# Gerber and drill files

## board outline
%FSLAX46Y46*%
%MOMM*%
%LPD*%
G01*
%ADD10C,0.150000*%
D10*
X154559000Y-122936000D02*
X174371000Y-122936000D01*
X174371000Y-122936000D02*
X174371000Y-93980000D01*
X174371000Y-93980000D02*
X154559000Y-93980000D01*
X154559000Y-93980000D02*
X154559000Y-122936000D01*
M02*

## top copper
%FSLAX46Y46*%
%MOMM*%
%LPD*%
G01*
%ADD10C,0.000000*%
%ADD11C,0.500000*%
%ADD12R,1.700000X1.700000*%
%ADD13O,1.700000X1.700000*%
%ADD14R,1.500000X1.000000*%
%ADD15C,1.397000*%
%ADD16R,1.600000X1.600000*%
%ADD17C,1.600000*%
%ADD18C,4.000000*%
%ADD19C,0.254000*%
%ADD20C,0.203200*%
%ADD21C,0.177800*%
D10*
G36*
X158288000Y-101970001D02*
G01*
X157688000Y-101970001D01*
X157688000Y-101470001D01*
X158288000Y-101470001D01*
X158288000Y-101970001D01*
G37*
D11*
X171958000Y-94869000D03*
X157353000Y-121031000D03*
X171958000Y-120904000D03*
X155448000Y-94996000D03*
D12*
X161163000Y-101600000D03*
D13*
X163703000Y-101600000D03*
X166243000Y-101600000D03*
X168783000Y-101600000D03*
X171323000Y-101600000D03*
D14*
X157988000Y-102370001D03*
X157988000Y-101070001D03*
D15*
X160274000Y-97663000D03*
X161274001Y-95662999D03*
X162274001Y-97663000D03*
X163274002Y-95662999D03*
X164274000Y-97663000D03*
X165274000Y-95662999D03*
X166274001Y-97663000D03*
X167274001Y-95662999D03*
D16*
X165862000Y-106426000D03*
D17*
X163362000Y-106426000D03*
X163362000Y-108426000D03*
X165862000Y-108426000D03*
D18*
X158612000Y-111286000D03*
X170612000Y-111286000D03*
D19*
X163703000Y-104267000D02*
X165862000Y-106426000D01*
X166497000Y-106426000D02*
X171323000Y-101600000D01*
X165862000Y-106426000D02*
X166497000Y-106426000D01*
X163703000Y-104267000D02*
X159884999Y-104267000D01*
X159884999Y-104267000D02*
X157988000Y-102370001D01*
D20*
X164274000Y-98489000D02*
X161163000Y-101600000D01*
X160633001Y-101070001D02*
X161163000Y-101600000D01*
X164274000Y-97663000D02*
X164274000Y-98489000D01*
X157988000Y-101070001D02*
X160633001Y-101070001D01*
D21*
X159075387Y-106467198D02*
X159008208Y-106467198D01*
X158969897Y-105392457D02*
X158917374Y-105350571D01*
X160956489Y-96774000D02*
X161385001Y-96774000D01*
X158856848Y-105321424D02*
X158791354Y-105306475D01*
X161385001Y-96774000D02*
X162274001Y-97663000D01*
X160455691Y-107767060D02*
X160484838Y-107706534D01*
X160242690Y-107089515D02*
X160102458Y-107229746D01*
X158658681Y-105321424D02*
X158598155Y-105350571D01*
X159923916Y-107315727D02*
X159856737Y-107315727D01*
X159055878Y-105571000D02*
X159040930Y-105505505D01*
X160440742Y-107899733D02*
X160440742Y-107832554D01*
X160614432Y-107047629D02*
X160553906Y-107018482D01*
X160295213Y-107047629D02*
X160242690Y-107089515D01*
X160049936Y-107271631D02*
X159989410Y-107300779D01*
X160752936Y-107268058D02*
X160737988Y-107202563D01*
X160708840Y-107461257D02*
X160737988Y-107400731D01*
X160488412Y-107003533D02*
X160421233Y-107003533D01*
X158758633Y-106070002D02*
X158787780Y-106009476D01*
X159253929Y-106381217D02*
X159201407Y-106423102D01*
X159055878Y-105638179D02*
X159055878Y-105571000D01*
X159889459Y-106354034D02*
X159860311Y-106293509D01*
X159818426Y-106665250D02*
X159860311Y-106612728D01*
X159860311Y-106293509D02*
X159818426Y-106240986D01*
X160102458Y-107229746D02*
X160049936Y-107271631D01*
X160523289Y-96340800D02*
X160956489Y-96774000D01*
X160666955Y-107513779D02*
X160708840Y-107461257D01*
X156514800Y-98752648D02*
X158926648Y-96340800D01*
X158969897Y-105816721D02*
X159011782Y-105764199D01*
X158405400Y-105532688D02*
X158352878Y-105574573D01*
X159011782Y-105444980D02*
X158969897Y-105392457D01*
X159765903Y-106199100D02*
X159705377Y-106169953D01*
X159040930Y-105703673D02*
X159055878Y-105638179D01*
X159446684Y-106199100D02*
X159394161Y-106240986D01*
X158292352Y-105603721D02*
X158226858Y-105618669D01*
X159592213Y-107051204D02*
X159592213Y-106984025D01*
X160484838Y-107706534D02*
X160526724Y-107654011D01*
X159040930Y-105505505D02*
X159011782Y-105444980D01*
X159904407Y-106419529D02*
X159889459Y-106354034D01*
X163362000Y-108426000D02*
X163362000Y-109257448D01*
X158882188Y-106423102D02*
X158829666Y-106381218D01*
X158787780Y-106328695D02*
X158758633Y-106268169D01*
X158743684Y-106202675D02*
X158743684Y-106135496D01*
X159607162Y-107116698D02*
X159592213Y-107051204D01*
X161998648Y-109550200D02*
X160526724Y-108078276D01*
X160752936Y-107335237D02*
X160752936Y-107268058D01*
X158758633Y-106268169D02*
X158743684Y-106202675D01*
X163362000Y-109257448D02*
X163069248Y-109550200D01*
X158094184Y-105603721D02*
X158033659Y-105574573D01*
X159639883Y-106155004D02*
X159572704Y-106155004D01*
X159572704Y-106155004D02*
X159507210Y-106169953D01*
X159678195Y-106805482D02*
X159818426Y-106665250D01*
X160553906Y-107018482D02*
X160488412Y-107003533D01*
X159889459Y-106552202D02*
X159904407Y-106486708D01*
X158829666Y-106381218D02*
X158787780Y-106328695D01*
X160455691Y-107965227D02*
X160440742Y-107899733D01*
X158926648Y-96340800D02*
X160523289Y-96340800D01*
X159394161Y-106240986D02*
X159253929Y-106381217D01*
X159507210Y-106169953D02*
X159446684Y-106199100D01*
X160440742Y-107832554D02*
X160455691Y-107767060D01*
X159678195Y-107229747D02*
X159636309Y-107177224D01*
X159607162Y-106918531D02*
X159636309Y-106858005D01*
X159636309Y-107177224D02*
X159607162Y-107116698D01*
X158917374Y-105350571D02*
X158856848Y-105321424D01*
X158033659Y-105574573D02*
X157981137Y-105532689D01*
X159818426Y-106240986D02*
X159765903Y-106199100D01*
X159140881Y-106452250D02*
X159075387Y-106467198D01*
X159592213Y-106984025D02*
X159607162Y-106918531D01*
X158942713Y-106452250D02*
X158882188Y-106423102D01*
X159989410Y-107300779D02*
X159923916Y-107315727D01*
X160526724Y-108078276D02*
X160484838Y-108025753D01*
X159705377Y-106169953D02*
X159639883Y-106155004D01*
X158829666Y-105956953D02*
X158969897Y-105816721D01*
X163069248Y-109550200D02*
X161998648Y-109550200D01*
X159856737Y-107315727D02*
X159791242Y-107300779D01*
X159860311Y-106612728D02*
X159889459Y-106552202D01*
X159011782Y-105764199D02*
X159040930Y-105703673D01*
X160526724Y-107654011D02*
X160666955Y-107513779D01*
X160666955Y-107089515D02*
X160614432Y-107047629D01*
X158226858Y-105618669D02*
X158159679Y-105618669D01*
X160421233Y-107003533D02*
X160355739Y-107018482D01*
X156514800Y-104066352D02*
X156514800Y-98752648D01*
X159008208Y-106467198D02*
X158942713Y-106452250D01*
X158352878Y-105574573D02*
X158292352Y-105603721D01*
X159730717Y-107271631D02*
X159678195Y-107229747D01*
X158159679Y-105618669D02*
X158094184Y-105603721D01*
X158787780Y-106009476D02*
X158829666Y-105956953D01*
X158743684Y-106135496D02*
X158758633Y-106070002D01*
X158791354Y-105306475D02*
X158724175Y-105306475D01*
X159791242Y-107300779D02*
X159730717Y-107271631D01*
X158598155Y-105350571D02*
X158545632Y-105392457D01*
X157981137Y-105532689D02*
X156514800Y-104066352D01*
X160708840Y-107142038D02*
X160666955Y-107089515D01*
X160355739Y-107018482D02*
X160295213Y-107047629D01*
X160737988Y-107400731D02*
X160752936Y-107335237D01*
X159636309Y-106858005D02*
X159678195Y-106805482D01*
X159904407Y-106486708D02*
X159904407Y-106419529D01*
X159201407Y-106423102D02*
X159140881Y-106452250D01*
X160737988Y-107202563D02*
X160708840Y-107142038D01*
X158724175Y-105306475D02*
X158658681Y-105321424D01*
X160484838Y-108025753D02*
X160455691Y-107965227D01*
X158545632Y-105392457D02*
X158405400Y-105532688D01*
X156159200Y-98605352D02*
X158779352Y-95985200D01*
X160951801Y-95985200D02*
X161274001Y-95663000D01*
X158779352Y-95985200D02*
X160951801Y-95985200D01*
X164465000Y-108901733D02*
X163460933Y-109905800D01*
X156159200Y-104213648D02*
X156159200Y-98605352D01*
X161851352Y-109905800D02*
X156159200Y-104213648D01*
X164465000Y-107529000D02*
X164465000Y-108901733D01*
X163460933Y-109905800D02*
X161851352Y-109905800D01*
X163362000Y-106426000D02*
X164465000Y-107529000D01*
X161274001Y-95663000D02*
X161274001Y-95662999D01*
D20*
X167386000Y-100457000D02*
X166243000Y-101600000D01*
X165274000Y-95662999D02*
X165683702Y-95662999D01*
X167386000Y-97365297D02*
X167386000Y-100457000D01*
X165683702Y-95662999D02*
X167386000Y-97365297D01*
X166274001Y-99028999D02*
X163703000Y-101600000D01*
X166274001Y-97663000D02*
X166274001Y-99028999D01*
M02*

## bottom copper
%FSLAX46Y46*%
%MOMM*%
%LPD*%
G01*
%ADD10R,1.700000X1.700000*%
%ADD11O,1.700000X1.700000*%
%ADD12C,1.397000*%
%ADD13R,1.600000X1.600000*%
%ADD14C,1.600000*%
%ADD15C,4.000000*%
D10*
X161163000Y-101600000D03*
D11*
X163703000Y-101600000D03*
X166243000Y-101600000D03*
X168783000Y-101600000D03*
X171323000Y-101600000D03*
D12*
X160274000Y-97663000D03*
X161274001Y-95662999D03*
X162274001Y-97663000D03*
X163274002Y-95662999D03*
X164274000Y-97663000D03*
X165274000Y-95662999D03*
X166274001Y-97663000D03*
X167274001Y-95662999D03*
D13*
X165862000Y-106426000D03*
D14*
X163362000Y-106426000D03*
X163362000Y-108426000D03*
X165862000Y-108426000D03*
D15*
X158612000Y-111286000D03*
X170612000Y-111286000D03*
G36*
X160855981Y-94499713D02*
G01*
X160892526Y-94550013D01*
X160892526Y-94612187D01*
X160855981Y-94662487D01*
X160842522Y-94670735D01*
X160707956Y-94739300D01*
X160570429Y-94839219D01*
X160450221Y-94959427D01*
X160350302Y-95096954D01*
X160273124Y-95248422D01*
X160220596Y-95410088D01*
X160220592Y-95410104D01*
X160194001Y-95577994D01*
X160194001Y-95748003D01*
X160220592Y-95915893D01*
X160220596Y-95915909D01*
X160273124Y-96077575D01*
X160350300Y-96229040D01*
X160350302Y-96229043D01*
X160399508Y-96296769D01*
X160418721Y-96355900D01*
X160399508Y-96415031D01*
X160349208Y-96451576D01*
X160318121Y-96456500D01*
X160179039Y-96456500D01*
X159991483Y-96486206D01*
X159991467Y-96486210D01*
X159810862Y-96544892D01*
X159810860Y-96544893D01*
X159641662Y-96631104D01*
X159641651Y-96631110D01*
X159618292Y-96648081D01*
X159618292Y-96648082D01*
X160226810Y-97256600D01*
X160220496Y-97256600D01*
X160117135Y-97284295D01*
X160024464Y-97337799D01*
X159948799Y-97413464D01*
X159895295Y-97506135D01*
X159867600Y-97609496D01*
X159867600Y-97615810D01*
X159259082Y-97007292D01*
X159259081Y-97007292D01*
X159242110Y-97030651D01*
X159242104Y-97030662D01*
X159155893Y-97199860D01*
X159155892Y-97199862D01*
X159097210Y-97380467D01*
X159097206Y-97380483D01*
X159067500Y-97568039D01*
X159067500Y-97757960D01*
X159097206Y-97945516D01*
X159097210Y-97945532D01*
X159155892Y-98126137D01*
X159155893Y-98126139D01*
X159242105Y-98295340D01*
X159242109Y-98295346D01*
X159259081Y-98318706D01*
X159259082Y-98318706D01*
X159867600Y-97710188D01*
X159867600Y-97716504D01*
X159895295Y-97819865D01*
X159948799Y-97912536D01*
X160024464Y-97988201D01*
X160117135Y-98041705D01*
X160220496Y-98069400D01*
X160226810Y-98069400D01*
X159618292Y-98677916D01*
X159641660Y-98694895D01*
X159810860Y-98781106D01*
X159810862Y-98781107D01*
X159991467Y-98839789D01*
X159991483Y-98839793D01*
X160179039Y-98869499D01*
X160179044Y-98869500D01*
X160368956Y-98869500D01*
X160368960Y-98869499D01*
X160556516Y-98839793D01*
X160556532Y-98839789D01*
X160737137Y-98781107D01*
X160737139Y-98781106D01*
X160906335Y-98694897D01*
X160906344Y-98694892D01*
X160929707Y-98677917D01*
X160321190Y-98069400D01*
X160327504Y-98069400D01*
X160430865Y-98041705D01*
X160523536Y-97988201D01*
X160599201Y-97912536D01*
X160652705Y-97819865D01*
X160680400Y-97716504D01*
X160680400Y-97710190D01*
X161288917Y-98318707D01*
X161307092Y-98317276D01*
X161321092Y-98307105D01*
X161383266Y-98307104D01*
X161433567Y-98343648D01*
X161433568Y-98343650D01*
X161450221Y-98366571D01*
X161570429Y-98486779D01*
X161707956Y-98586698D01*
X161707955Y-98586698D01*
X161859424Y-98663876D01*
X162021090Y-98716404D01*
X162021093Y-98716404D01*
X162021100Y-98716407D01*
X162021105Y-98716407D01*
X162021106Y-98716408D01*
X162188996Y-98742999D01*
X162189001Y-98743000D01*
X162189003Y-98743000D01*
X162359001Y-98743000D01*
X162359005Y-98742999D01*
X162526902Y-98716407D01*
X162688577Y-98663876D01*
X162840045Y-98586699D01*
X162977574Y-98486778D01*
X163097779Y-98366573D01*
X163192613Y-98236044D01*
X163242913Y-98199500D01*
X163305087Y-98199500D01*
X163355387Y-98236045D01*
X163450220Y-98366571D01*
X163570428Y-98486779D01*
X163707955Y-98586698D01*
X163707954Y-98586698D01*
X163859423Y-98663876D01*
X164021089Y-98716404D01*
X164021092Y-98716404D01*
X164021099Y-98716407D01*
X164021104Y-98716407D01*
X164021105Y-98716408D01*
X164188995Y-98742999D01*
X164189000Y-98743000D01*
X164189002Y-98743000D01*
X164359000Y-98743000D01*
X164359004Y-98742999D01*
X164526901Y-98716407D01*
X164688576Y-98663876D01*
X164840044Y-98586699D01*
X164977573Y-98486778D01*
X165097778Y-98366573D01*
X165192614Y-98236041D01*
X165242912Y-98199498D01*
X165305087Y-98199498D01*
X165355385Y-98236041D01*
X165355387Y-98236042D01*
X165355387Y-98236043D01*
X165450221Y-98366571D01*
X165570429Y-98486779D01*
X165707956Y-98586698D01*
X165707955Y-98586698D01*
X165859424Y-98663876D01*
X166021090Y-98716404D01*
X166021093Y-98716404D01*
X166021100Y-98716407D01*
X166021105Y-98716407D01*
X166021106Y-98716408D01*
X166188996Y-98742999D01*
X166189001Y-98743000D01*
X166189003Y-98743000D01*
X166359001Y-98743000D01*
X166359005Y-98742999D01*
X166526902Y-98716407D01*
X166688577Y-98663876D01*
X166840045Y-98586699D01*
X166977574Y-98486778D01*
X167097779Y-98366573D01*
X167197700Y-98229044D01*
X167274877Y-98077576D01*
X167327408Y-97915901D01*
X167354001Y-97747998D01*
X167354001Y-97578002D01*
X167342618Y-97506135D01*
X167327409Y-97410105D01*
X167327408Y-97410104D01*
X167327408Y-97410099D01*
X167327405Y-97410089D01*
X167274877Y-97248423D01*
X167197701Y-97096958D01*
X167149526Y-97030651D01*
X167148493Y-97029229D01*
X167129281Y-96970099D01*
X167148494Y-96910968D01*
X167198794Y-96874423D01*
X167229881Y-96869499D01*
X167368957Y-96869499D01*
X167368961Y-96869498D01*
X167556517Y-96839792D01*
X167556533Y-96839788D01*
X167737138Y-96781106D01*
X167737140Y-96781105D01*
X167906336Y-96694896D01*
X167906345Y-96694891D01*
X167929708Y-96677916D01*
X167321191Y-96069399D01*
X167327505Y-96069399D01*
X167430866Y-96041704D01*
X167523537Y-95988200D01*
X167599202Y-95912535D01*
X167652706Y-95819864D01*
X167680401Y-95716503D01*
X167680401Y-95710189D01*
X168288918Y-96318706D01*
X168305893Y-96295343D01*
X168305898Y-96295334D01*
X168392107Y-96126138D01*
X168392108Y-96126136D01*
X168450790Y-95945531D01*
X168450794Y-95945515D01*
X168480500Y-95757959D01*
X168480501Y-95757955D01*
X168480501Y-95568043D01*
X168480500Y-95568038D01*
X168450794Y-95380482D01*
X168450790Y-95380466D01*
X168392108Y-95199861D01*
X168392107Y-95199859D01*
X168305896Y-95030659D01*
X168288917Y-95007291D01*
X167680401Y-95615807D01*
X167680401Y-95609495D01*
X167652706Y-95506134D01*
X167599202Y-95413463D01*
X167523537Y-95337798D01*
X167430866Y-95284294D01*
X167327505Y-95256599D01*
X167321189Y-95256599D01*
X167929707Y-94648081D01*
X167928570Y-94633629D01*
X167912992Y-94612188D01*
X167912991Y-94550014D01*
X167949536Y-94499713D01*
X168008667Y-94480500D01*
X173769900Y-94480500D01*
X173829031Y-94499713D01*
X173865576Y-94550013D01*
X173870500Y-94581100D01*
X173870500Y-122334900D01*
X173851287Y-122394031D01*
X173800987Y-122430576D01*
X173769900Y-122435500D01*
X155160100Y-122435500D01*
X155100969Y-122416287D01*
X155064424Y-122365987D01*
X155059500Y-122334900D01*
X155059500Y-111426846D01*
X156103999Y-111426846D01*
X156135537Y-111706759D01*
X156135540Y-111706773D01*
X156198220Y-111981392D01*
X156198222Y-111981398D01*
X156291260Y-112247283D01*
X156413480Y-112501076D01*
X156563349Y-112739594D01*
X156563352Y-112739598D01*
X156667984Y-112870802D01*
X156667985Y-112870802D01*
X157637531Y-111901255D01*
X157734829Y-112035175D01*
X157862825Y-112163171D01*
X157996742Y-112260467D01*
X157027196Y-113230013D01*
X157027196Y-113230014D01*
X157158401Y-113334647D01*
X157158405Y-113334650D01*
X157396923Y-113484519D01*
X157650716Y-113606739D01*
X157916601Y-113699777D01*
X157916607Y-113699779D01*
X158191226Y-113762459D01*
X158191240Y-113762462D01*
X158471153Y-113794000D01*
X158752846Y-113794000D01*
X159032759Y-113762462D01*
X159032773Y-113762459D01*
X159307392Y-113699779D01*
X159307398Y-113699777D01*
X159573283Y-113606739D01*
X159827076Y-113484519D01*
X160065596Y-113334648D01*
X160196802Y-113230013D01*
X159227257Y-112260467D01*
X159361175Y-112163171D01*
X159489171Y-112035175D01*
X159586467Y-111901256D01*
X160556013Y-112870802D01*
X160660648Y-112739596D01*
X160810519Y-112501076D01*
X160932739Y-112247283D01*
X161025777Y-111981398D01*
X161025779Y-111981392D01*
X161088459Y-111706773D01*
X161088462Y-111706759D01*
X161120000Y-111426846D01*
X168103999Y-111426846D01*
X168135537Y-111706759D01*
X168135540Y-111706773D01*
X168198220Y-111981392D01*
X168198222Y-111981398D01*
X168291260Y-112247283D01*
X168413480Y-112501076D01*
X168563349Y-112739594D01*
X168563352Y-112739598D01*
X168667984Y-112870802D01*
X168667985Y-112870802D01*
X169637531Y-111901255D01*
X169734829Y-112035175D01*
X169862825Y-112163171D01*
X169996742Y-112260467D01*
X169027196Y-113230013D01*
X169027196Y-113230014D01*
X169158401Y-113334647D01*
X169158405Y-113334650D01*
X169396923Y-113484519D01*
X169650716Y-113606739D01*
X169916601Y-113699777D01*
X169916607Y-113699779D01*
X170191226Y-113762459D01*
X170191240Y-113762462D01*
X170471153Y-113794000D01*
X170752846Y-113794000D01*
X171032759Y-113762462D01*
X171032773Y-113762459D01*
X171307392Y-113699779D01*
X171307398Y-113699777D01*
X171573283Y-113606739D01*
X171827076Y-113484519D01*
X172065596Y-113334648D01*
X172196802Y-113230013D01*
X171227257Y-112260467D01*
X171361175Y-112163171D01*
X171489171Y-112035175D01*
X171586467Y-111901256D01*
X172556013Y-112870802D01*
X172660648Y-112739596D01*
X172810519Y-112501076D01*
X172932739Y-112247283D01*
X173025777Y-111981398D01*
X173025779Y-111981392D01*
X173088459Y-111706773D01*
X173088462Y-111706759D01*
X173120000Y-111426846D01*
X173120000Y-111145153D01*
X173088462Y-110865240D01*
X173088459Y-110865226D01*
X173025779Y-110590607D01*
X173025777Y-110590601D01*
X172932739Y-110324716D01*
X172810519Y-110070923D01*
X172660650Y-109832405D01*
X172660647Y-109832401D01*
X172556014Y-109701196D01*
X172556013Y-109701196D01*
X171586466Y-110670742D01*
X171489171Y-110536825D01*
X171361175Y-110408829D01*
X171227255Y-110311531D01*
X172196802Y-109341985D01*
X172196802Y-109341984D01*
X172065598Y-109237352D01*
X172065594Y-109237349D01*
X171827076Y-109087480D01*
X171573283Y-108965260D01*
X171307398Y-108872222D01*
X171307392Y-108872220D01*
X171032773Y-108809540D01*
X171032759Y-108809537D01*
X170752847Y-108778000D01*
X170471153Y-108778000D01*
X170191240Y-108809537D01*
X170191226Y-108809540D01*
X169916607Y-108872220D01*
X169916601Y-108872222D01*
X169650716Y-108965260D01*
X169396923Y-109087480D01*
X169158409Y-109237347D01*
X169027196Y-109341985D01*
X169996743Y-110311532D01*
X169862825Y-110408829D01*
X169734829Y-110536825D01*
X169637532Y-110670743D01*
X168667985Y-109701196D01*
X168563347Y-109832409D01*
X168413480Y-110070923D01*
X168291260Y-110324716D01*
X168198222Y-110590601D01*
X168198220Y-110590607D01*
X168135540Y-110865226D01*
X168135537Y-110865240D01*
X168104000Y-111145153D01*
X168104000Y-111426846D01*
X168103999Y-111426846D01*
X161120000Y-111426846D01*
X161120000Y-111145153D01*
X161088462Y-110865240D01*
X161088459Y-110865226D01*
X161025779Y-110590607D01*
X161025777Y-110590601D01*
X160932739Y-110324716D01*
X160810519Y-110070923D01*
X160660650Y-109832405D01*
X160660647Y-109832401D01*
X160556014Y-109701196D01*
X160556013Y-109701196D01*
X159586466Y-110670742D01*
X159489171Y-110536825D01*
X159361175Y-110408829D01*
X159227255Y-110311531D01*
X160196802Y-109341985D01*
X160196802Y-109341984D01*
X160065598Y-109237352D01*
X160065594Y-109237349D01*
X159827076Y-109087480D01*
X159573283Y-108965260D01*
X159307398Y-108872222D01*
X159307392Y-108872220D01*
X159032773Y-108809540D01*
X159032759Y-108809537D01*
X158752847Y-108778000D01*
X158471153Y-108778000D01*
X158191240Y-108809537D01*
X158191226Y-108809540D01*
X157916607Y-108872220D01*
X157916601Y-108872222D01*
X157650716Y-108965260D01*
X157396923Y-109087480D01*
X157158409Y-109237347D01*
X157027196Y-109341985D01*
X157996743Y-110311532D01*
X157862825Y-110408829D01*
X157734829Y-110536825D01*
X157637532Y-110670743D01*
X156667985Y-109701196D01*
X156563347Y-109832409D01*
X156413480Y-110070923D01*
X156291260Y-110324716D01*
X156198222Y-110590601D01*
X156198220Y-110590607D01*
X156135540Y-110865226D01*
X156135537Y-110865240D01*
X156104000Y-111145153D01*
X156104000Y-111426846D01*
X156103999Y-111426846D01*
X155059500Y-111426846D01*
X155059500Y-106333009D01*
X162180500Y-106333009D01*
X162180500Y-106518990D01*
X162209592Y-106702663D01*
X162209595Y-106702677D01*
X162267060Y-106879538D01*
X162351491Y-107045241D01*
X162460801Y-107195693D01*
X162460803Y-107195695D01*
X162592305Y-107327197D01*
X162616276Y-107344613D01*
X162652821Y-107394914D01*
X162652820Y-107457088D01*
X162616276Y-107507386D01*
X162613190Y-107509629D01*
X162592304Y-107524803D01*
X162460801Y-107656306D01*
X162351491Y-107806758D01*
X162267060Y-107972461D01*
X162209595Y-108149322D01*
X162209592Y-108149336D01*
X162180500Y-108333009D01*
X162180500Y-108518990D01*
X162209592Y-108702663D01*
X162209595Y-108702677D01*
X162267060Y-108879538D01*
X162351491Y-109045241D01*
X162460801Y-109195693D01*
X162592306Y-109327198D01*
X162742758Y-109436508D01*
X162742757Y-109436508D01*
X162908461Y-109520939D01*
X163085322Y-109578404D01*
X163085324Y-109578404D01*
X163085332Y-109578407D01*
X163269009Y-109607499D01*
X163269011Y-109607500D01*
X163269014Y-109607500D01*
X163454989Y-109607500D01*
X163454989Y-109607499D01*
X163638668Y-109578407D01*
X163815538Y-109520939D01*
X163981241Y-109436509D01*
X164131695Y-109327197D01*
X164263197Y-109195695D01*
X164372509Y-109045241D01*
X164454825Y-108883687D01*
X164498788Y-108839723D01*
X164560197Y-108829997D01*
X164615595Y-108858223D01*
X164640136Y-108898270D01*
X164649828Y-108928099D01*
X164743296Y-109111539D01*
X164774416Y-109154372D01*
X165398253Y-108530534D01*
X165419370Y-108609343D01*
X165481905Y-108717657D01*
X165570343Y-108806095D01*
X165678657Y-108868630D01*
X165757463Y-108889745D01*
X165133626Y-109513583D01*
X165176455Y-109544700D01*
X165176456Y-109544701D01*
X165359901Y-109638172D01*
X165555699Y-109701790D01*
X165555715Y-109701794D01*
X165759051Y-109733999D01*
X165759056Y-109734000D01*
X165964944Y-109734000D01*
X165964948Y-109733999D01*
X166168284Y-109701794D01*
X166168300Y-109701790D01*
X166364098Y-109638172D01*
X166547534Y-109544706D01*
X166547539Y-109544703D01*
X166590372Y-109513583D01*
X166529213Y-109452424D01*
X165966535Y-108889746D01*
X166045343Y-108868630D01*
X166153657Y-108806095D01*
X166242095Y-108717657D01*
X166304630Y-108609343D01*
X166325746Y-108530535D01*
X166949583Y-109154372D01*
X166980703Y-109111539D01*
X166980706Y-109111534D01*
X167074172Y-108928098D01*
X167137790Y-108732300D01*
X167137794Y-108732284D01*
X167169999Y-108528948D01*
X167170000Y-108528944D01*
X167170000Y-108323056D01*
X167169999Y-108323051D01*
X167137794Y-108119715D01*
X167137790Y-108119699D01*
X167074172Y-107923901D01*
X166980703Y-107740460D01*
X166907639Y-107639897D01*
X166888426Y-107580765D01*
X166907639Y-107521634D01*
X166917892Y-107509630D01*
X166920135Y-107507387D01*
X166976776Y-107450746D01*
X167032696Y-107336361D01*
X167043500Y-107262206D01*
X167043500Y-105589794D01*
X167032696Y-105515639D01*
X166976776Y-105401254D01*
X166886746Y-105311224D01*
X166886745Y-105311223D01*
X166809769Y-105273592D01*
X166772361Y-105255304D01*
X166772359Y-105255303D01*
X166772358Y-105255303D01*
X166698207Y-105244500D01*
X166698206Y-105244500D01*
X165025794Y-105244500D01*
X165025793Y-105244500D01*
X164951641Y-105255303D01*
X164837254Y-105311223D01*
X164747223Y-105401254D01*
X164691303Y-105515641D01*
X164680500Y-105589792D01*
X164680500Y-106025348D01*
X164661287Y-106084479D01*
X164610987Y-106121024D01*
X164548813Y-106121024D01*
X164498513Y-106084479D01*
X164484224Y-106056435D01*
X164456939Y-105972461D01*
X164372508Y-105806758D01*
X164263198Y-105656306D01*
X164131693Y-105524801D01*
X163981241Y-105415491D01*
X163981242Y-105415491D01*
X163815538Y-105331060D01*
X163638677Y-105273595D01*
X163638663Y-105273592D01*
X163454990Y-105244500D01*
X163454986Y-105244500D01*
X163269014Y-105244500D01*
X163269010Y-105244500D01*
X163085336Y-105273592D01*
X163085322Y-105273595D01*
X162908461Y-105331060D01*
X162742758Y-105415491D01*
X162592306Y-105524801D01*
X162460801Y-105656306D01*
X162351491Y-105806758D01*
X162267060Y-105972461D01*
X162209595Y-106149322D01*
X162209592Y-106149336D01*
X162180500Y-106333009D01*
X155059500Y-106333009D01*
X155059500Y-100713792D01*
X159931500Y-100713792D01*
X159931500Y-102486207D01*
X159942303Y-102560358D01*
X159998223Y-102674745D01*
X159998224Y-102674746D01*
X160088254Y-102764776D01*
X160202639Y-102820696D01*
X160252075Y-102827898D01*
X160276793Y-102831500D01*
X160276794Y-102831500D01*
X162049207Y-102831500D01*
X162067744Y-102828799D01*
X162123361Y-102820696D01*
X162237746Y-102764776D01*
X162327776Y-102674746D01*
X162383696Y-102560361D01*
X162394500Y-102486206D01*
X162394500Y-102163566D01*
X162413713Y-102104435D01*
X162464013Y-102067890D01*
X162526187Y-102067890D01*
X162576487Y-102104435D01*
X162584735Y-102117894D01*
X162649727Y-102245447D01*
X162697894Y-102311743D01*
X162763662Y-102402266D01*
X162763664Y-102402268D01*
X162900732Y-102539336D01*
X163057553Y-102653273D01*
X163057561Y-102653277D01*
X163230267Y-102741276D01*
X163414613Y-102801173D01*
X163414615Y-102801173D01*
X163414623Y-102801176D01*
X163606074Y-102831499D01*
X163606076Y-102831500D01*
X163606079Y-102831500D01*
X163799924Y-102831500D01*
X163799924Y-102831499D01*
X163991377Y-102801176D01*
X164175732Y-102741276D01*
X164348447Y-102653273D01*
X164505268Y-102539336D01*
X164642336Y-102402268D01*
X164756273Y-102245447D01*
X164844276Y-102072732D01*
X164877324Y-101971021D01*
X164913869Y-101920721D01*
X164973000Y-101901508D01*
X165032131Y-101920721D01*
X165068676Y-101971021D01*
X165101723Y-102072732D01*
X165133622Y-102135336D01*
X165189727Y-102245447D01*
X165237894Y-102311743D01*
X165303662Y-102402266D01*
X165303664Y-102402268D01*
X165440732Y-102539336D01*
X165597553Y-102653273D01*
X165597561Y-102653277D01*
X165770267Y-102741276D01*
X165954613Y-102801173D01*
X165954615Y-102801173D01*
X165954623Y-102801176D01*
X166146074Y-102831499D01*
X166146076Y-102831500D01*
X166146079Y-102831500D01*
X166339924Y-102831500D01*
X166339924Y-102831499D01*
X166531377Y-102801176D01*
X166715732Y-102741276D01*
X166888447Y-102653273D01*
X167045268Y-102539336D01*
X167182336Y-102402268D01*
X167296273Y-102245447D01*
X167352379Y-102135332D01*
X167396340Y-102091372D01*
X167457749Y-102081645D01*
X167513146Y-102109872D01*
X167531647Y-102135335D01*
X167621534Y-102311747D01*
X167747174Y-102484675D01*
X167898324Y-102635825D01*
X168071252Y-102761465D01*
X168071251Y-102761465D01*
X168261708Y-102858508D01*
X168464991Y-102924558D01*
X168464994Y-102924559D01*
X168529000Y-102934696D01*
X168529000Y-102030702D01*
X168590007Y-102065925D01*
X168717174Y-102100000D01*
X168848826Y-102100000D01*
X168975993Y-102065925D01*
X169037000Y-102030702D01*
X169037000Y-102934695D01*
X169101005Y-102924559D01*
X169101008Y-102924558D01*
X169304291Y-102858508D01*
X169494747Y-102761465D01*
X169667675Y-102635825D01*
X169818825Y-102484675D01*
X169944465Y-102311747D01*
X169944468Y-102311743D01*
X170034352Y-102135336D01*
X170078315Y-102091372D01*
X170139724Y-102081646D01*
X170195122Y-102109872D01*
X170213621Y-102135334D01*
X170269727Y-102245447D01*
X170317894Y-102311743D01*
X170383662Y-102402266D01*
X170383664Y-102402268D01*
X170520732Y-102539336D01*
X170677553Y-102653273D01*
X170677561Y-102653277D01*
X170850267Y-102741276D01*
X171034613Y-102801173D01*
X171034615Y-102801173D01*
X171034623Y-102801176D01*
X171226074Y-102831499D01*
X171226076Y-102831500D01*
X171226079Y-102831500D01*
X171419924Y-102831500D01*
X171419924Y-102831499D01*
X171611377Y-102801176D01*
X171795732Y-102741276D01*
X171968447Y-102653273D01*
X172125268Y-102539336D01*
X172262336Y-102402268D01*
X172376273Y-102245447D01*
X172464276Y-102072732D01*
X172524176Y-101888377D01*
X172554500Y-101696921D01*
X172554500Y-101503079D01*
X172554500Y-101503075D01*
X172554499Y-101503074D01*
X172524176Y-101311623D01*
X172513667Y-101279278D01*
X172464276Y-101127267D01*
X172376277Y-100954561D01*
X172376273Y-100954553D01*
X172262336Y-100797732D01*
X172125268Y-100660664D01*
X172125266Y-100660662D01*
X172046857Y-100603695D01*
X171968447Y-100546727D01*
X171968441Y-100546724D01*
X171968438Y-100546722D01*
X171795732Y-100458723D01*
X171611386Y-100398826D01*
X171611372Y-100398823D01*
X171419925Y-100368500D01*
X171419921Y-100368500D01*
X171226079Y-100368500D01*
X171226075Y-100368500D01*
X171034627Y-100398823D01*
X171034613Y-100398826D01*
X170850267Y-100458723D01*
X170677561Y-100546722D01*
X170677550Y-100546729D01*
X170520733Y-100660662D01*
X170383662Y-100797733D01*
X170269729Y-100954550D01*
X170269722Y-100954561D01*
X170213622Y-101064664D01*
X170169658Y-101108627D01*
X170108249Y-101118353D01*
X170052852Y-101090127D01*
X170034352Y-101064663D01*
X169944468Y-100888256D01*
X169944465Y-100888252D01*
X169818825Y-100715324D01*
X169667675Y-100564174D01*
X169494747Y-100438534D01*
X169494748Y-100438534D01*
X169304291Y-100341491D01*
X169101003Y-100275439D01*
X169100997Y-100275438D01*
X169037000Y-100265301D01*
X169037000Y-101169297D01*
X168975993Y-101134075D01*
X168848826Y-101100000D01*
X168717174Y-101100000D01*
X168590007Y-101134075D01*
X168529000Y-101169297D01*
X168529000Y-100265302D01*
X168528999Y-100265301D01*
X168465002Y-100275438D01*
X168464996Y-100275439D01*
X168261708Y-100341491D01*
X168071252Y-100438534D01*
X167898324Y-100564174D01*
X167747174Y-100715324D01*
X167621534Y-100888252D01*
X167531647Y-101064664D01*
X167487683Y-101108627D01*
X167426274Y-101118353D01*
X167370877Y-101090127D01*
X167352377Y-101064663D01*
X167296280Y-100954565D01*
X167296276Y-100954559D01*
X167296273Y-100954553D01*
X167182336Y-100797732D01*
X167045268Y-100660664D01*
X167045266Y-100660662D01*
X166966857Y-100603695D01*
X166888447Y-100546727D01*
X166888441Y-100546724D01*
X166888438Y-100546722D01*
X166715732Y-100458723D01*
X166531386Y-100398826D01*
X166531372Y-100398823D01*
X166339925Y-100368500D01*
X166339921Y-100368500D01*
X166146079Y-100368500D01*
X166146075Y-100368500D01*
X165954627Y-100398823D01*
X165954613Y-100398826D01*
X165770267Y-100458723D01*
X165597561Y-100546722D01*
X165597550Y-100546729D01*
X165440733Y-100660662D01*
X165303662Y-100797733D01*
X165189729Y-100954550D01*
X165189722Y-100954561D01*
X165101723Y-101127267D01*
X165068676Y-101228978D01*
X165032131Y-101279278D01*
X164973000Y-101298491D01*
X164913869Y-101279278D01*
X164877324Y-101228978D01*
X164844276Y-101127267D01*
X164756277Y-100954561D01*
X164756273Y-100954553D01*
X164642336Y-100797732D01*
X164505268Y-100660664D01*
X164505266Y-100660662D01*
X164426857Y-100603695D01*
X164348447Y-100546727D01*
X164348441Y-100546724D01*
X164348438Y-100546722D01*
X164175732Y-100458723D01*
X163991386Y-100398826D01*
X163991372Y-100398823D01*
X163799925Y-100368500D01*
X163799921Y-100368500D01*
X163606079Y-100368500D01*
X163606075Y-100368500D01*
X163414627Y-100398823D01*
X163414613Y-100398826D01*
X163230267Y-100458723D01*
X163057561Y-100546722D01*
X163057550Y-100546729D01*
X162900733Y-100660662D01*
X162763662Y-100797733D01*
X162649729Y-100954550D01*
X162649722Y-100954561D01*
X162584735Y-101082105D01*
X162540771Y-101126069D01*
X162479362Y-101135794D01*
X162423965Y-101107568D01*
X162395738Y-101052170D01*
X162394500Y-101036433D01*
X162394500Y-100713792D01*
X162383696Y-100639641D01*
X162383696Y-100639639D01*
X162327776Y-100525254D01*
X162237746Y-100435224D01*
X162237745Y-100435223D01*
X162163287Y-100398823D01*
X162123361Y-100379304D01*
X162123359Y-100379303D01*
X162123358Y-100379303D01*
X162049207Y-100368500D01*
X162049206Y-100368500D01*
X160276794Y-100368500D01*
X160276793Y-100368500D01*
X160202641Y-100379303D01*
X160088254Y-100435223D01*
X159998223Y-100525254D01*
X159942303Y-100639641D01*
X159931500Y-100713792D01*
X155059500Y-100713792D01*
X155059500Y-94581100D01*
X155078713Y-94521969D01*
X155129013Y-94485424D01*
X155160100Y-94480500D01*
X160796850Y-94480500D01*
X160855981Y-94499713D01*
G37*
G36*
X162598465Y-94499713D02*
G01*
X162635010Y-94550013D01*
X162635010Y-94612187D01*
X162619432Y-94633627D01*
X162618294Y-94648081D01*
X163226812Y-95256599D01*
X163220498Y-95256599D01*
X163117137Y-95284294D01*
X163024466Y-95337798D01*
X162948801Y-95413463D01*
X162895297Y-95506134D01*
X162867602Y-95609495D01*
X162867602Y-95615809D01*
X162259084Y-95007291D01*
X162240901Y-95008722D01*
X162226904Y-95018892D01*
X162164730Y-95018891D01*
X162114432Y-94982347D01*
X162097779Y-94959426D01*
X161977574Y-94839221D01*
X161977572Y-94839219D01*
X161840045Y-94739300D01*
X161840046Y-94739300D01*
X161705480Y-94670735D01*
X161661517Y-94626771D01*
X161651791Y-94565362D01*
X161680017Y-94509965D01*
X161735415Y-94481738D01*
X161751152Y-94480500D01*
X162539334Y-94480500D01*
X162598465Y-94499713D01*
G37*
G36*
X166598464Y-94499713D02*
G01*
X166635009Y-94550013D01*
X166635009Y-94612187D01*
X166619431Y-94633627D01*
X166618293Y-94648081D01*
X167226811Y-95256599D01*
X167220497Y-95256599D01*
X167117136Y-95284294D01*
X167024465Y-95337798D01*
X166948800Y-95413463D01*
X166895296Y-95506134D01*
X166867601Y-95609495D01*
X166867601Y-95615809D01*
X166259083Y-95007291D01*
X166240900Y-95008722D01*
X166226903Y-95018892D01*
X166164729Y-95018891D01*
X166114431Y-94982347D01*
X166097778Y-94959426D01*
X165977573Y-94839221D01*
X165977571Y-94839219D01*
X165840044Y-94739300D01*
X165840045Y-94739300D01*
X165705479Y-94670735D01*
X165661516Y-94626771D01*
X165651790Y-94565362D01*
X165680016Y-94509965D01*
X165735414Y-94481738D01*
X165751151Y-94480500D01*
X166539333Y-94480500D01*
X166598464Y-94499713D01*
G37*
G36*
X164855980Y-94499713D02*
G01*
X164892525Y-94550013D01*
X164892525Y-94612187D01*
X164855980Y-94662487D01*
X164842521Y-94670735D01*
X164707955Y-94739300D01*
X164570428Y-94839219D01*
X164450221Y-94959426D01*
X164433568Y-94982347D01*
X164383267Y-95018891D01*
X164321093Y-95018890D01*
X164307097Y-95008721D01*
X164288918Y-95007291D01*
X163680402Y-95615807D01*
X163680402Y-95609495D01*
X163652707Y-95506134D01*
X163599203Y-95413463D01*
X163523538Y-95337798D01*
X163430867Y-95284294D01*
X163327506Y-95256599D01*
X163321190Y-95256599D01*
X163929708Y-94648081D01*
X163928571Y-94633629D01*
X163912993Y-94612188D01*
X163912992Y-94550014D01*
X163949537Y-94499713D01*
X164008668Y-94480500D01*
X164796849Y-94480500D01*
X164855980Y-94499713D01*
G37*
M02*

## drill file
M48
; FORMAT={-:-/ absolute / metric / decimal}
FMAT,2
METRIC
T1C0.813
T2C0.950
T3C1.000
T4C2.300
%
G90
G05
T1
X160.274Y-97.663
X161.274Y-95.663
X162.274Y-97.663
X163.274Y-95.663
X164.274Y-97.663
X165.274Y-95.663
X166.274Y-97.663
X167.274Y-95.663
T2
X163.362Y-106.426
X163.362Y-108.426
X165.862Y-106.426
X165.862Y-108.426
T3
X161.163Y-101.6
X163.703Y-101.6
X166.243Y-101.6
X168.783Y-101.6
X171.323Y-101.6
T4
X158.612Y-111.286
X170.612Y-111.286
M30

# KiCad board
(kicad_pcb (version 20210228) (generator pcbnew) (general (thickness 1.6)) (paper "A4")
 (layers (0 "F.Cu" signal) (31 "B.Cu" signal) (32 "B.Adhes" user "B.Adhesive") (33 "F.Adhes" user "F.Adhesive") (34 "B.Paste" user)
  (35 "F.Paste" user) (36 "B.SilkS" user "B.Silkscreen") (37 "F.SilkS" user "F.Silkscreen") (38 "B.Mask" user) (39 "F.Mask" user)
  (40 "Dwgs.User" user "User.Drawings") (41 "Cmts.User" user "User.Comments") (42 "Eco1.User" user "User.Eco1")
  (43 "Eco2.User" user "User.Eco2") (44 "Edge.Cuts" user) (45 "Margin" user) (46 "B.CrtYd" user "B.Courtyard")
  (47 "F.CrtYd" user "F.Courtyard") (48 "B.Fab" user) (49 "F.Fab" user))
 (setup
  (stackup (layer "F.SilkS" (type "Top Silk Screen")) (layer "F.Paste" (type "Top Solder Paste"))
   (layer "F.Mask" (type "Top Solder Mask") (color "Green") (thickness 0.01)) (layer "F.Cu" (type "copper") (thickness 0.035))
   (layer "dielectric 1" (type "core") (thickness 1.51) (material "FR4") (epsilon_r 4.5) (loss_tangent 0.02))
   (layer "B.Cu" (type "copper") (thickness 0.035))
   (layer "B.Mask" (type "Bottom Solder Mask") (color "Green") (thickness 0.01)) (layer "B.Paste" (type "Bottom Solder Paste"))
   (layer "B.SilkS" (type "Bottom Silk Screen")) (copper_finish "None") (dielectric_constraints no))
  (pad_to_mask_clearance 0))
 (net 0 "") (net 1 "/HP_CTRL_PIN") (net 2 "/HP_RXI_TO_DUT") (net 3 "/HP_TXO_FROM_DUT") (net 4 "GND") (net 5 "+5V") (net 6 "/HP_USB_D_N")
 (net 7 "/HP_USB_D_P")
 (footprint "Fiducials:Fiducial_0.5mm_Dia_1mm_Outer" (layer "F.Cu") (at 171.958 94.869)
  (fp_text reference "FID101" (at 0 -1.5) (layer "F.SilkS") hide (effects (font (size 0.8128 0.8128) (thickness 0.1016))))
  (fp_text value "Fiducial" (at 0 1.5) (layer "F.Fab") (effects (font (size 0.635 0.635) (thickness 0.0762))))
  (pad "~" smd circle (at 0 0) (locked) (size 0.5 0.5) (layers "F.Cu" "F.Mask") (solder_mask_margin 0.25) (clearance 0.25)))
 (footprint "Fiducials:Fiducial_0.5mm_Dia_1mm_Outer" (layer "F.Cu") (at 157.353 121.031)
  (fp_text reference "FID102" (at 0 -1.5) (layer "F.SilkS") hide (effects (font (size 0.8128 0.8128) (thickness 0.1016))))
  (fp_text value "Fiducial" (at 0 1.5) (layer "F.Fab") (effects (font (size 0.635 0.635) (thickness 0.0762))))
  (pad "~" smd circle (at 0 0) (locked) (size 0.5 0.5) (layers "F.Cu" "F.Mask") (solder_mask_margin 0.25) (clearance 0.25)))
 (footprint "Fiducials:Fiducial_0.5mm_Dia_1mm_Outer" (layer "F.Cu") (at 171.958 120.904)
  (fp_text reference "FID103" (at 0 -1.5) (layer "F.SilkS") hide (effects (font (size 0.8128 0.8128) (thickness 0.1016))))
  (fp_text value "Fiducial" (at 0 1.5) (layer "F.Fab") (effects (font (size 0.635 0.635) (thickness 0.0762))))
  (pad "~" smd circle (at 0 0) (locked) (size 0.5 0.5) (layers "F.Cu" "F.Mask") (solder_mask_margin 0.25) (clearance 0.25)))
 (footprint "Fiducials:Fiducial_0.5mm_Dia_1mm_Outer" (layer "F.Cu") (at 155.448 94.996)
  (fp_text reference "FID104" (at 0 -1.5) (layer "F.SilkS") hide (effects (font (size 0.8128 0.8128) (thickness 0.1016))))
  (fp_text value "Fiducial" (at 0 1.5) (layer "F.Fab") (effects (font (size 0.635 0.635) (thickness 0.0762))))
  (pad "~" smd circle (at 0 0) (locked) (size 0.5 0.5) (layers "F.Cu" "F.Mask") (solder_mask_margin 0.25) (clearance 0.25)))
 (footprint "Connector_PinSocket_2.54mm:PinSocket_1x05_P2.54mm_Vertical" (layer "F.Cu") (at 161.163 101.6 90)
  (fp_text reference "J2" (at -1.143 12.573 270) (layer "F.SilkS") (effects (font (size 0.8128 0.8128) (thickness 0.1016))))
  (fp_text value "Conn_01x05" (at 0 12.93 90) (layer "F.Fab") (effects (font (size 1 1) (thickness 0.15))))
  (pad "1" thru_hole rect (at 0 0 90) (locked) (size 1.7 1.7) (drill 1) (layers *.Cu *.Mask) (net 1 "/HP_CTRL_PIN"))
  (pad "2" thru_hole oval (at 0 2.54 90) (locked) (size 1.7 1.7) (drill 1) (layers *.Cu *.Mask) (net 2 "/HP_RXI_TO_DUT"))
  (pad "3" thru_hole oval (at 0 5.08 90) (locked) (size 1.7 1.7) (drill 1) (layers *.Cu *.Mask) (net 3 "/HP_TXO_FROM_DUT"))
  (pad "4" thru_hole oval (at 0 7.62 90) (locked) (size 1.7 1.7) (drill 1) (layers *.Cu *.Mask) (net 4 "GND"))
  (pad "5" thru_hole oval (at 0 10.16 90) (locked) (size 1.7 1.7) (drill 1) (layers *.Cu *.Mask) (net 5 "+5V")))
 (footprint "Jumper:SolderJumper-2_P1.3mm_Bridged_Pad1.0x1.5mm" (layer "F.Cu") (at 157.988 101.720001 90)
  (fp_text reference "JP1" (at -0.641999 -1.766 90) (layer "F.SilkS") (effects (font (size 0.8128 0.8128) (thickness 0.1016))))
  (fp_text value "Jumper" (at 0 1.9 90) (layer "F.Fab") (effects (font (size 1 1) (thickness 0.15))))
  (fp_poly (pts (xy -0.25 -0.3) (xy 0.25 -0.3) (xy 0.25 0.3) (xy -0.25 0.3)) (layer "F.Cu") (width 0) (fill solid))
  (pad "1" smd rect (at -0.65 0 90) (locked) (size 1 1.5) (layers "F.Cu" "F.Mask") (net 5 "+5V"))
  (pad "2" smd rect (at 0.65 0 90) (locked) (size 1 1.5) (layers "F.Cu" "F.Mask") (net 1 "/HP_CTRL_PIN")))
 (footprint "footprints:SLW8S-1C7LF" (layer "F.Cu") (at 160.274 97.663)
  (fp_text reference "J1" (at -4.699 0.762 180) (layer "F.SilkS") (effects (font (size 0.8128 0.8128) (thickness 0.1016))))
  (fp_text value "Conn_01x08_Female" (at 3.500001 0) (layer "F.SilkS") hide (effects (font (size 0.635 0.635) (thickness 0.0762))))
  (pad "1" thru_hole circle (at 0 0) (locked) (size 1.397 1.397) (drill 0.8128) (layers *.Cu *.Mask) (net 4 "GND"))
  (pad "2" thru_hole circle (at 1.000001 -2.000001) (locked) (size 1.397 1.397) (drill 0.8128) (layers *.Cu *.Mask) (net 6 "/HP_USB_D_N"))
  (pad "3" thru_hole circle (at 2.000001 0) (locked) (size 1.397 1.397) (drill 0.8128) (layers *.Cu *.Mask) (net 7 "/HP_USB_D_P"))
  (pad "4" thru_hole circle (at 3.000002 -2.000001) (locked) (size 1.397 1.397) (drill 0.8128) (layers *.Cu *.Mask) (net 4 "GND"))
  (pad "5" thru_hole circle (at 4 0) (locked) (size 1.397 1.397) (drill 0.8128) (layers *.Cu *.Mask) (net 1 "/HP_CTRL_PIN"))
  (pad "6" thru_hole circle (at 5 -2.000001) (locked) (size 1.397 1.397) (drill 0.8128) (layers *.Cu *.Mask) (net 3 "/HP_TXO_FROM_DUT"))
  (pad "7" thru_hole circle (at 6.000001 0) (locked) (size 1.397 1.397) (drill 0.8128) (layers *.Cu *.Mask) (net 2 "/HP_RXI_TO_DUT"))
  (pad "8" thru_hole circle (at 7.000001 -2.000001) (locked) (size 1.397 1.397) (drill 0.8128) (layers *.Cu *.Mask) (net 4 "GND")))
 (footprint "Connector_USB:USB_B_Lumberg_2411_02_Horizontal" (layer "F.Cu") (at 165.862 106.426 -90)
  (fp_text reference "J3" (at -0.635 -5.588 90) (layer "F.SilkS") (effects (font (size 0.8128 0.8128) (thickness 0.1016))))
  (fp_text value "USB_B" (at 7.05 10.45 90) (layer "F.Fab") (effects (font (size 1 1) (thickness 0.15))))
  (pad "1" thru_hole rect (at 0 0) (locked) (size 1.6 1.6) (drill 0.95) (layers *.Cu *.Mask) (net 5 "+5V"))
  (pad "2" thru_hole circle (at 0 2.5) (locked) (size 1.6 1.6) (drill 0.95) (layers *.Cu *.Mask) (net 6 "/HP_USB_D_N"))
  (pad "3" thru_hole circle (at 2 2.5) (locked) (size 1.6 1.6) (drill 0.95) (layers *.Cu *.Mask) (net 7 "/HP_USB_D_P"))
  (pad "4" thru_hole circle (at 2 0) (locked) (size 1.6 1.6) (drill 0.95) (layers *.Cu *.Mask) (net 4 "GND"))
  (pad "5" thru_hole circle (at 4.86 7.25) (locked) (size 4 4) (drill 2.3) (layers *.Cu *.Mask) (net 4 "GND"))
  (pad "5" thru_hole circle (at 4.86 -4.75) (locked) (size 4 4) (drill 2.3) (layers *.Cu *.Mask) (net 4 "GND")))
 (gr_line (start 154.559 122.936) (end 174.371 122.936) (layer "Edge.Cuts") (width 0.15))
 (gr_line (start 174.371 122.936) (end 174.371 93.98) (layer "Edge.Cuts") (width 0.15))
 (gr_line (start 174.371 93.98) (end 154.559 93.98) (layer "Edge.Cuts") (width 0.15))
 (gr_line (start 154.559 93.98) (end 154.559 122.936) (layer "Edge.Cuts") (width 0.15))
 (segment (start 163.703 104.267) (end 165.862 106.426) (width 0.254) (layer "F.Cu") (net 5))
 (segment (start 166.497 106.426) (end 171.323 101.6) (width 0.254) (layer "F.Cu") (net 5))
 (segment (start 165.862 106.426) (end 166.497 106.426) (width 0.254) (layer "F.Cu") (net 5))
 (segment (start 163.703 104.267) (end 159.884999 104.267) (width 0.254) (layer "F.Cu") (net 5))
 (segment (start 159.884999 104.267) (end 157.988 102.370001) (width 0.254) (layer "F.Cu") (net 5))
 (segment (start 164.274 98.489) (end 161.163 101.6) (width 0.2032) (layer "F.Cu") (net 1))
 (segment (start 160.633001 101.070001) (end 161.163 101.6) (width 0.2032) (layer "F.Cu") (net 1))
 (segment (start 164.274 97.663) (end 164.274 98.489) (width 0.2032) (layer "F.Cu") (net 1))
 (segment (start 157.988 101.070001) (end 160.633001 101.070001) (width 0.2032) (layer "F.Cu") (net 1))
 (segment (start 159.075387 106.467198) (end 159.008208 106.467198) (width 0.1778) (layer "F.Cu") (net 7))
 (segment (start 158.969897 105.392457) (end 158.917374 105.350571) (width 0.1778) (layer "F.Cu") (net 7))
 (segment (start 160.956489 96.774) (end 161.385001 96.774) (width 0.1778) (layer "F.Cu") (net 7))
 (segment (start 158.856848 105.321424) (end 158.791354 105.306475) (width 0.1778) (layer "F.Cu") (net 7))
 (segment (start 161.385001 96.774) (end 162.274001 97.663) (width 0.1778) (layer "F.Cu") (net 7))
 (segment (start 160.455691 107.76706) (end 160.484838 107.706534) (width 0.1778) (layer "F.Cu") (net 7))
 (segment (start 160.24269 107.089515) (end 160.102458 107.229746) (width 0.1778) (layer "F.Cu") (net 7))
 (segment (start 158.658681 105.321424) (end 158.598155 105.350571) (width 0.1778) (layer "F.Cu") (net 7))
 (segment (start 159.923916 107.315727) (end 159.856737 107.315727) (width 0.1778) (layer "F.Cu") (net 7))
 (segment (start 159.055878 105.571) (end 159.04093 105.505505) (width 0.1778) (layer "F.Cu") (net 7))
 (segment (start 160.440742 107.899733) (end 160.440742 107.832554) (width 0.1778) (layer "F.Cu") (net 7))
 (segment (start 160.614432 107.047629) (end 160.553906 107.018482) (width 0.1778) (layer "F.Cu") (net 7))
 (segment (start 160.295213 107.047629) (end 160.24269 107.089515) (width 0.1778) (layer "F.Cu") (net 7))
 (segment (start 160.049936 107.271631) (end 159.98941 107.300779) (width 0.1778) (layer "F.Cu") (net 7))
 (segment (start 160.752936 107.268058) (end 160.737988 107.202563) (width 0.1778) (layer "F.Cu") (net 7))
 (segment (start 160.70884 107.461257) (end 160.737988 107.400731) (width 0.1778) (layer "F.Cu") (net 7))
 (segment (start 160.488412 107.003533) (end 160.421233 107.003533) (width 0.1778) (layer "F.Cu") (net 7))
 (segment (start 158.758633 106.070002) (end 158.78778 106.009476) (width 0.1778) (layer "F.Cu") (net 7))
 (segment (start 159.253929 106.381217) (end 159.201407 106.423102) (width 0.1778) (layer "F.Cu") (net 7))
 (segment (start 159.055878 105.638179) (end 159.055878 105.571) (width 0.1778) (layer "F.Cu") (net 7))
 (segment (start 159.889459 106.354034) (end 159.860311 106.293509) (width 0.1778) (layer "F.Cu") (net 7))
 (segment (start 159.818426 106.66525) (end 159.860311 106.612728) (width 0.1778) (layer "F.Cu") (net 7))
 (segment (start 159.860311 106.293509) (end 159.818426 106.240986) (width 0.1778) (layer "F.Cu") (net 7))
 (segment (start 160.102458 107.229746) (end 160.049936 107.271631) (width 0.1778) (layer "F.Cu") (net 7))
 (segment (start 160.523289 96.3408) (end 160.956489 96.774) (width 0.1778) (layer "F.Cu") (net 7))
 (segment (start 160.666955 107.513779) (end 160.70884 107.461257) (width 0.1778) (layer "F.Cu") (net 7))
 (segment (start 156.5148 98.752648) (end 158.926648 96.3408) (width 0.1778) (layer "F.Cu") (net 7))
 (segment (start 158.969897 105.816721) (end 159.011782 105.764199) (width 0.1778) (layer "F.Cu") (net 7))
 (segment (start 158.4054 105.532688) (end 158.352878 105.574573) (width 0.1778) (layer "F.Cu") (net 7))
 (segment (start 159.011782 105.44498) (end 158.969897 105.392457) (width 0.1778) (layer "F.Cu") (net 7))
 (segment (start 159.765903 106.1991) (end 159.705377 106.169953) (width 0.1778) (layer "F.Cu") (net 7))
 (segment (start 159.04093 105.703673) (end 159.055878 105.638179) (width 0.1778) (layer "F.Cu") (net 7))
 (segment (start 159.446684 106.1991) (end 159.394161 106.240986) (width 0.1778) (layer "F.Cu") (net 7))
 (segment (start 158.292352 105.603721) (end 158.226858 105.618669) (width 0.1778) (layer "F.Cu") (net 7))
 (segment (start 159.592213 107.051204) (end 159.592213 106.984025) (width 0.1778) (layer "F.Cu") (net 7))
 (segment (start 160.484838 107.706534) (end 160.526724 107.654011) (width 0.1778) (layer "F.Cu") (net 7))
 (segment (start 159.04093 105.505505) (end 159.011782 105.44498) (width 0.1778) (layer "F.Cu") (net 7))
 (segment (start 159.904407 106.419529) (end 159.889459 106.354034) (width 0.1778) (layer "F.Cu") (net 7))
 (segment (start 163.362 108.426) (end 163.362 109.257448) (width 0.1778) (layer "F.Cu") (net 7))
 (segment (start 158.882188 106.423102) (end 158.829666 106.381218) (width 0.1778) (layer "F.Cu") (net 7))
 (segment (start 158.78778 106.328695) (end 158.758633 106.268169) (width 0.1778) (layer "F.Cu") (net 7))
 (segment (start 158.743684 106.202675) (end 158.743684 106.135496) (width 0.1778) (layer "F.Cu") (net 7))
 (segment (start 159.607162 107.116698) (end 159.592213 107.051204) (width 0.1778) (layer "F.Cu") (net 7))
 (segment (start 161.998648 109.5502) (end 160.526724 108.078276) (width 0.1778) (layer "F.Cu") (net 7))
 (segment (start 160.752936 107.335237) (end 160.752936 107.268058) (width 0.1778) (layer "F.Cu") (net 7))
 (segment (start 158.758633 106.268169) (end 158.743684 106.202675) (width 0.1778) (layer "F.Cu") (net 7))
 (segment (start 163.362 109.257448) (end 163.069248 109.5502) (width 0.1778) (layer "F.Cu") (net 7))
 (segment (start 158.094184 105.603721) (end 158.033659 105.574573) (width 0.1778) (layer "F.Cu") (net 7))
 (segment (start 159.639883 106.155004) (end 159.572704 106.155004) (width 0.1778) (layer "F.Cu") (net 7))
 (segment (start 159.572704 106.155004) (end 159.50721 106.169953) (width 0.1778) (layer "F.Cu") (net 7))
 (segment (start 159.678195 106.805482) (end 159.818426 106.66525) (width 0.1778) (layer "F.Cu") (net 7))
 (segment (start 160.553906 107.018482) (end 160.488412 107.003533) (width 0.1778) (layer "F.Cu") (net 7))
 (segment (start 159.889459 106.552202) (end 159.904407 106.486708) (width 0.1778) (layer "F.Cu") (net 7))
 (segment (start 158.829666 106.381218) (end 158.78778 106.328695) (width 0.1778) (layer "F.Cu") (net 7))
 (segment (start 160.455691 107.965227) (end 160.440742 107.899733) (width 0.1778) (layer "F.Cu") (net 7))
 (segment (start 158.926648 96.3408) (end 160.523289 96.3408) (width 0.1778) (layer "F.Cu") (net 7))
 (segment (start 159.394161 106.240986) (end 159.253929 106.381217) (width 0.1778) (layer "F.Cu") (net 7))
 (segment (start 159.50721 106.169953) (end 159.446684 106.1991) (width 0.1778) (layer "F.Cu") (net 7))
 (segment (start 160.440742 107.832554) (end 160.455691 107.76706) (width 0.1778) (layer "F.Cu") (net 7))
 (segment (start 159.678195 107.229747) (end 159.636309 107.177224) (width 0.1778) (layer "F.Cu") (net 7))
 (segment (start 159.607162 106.918531) (end 159.636309 106.858005) (width 0.1778) (layer "F.Cu") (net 7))
 (segment (start 159.636309 107.177224) (end 159.607162 107.116698) (width 0.1778) (layer "F.Cu") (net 7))
 (segment (start 158.917374 105.350571) (end 158.856848 105.321424) (width 0.1778) (layer "F.Cu") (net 7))
 (segment (start 158.033659 105.574573) (end 157.981137 105.532689) (width 0.1778) (layer "F.Cu") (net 7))
 (segment (start 159.818426 106.240986) (end 159.765903 106.1991) (width 0.1778) (layer "F.Cu") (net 7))
 (segment (start 159.140881 106.45225) (end 159.075387 106.467198) (width 0.1778) (layer "F.Cu") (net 7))
 (segment (start 159.592213 106.984025) (end 159.607162 106.918531) (width 0.1778) (layer "F.Cu") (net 7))
 (segment (start 158.942713 106.45225) (end 158.882188 106.423102) (width 0.1778) (layer "F.Cu") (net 7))
 (segment (start 159.98941 107.300779) (end 159.923916 107.315727) (width 0.1778) (layer "F.Cu") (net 7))
 (segment (start 160.526724 108.078276) (end 160.484838 108.025753) (width 0.1778) (layer "F.Cu") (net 7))
 (segment (start 159.705377 106.169953) (end 159.639883 106.155004) (width 0.1778) (layer "F.Cu") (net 7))
 (segment (start 158.829666 105.956953) (end 158.969897 105.816721) (width 0.1778) (layer "F.Cu") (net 7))
 (segment (start 163.069248 109.5502) (end 161.998648 109.5502) (width 0.1778) (layer "F.Cu") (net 7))
 (segment (start 159.856737 107.315727) (end 159.791242 107.300779) (width 0.1778) (layer "F.Cu") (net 7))
 (segment (start 159.860311 106.612728) (end 159.889459 106.552202) (width 0.1778) (layer "F.Cu") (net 7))
 (segment (start 159.011782 105.764199) (end 159.04093 105.703673) (width 0.1778) (layer "F.Cu") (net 7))
 (segment (start 160.526724 107.654011) (end 160.666955 107.513779) (width 0.1778) (layer "F.Cu") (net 7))
 (segment (start 160.666955 107.089515) (end 160.614432 107.047629) (width 0.1778) (layer "F.Cu") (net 7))
 (segment (start 158.226858 105.618669) (end 158.159679 105.618669) (width 0.1778) (layer "F.Cu") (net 7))
 (segment (start 160.421233 107.003533) (end 160.355739 107.018482) (width 0.1778) (layer "F.Cu") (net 7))
 (segment (start 156.5148 104.066352) (end 156.5148 98.752648) (width 0.1778) (layer "F.Cu") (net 7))
 (segment (start 159.008208 106.467198) (end 158.942713 106.45225) (width 0.1778) (layer "F.Cu") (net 7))
 (segment (start 158.352878 105.574573) (end 158.292352 105.603721) (width 0.1778) (layer "F.Cu") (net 7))
 (segment (start 159.730717 107.271631) (end 159.678195 107.229747) (width 0.1778) (layer "F.Cu") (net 7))
 (segment (start 158.159679 105.618669) (end 158.094184 105.603721) (width 0.1778) (layer "F.Cu") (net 7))
 (segment (start 158.78778 106.009476) (end 158.829666 105.956953) (width 0.1778) (layer "F.Cu") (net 7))
 (segment (start 158.743684 106.135496) (end 158.758633 106.070002) (width 0.1778) (layer "F.Cu") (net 7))
 (segment (start 158.791354 105.306475) (end 158.724175 105.306475) (width 0.1778) (layer "F.Cu") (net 7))
 (segment (start 159.791242 107.300779) (end 159.730717 107.271631) (width 0.1778) (layer "F.Cu") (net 7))
 (segment (start 158.598155 105.350571) (end 158.545632 105.392457) (width 0.1778) (layer "F.Cu") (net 7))
 (segment (start 157.981137 105.532689) (end 156.5148 104.066352) (width 0.1778) (layer "F.Cu") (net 7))
 (segment (start 160.70884 107.142038) (end 160.666955 107.089515) (width 0.1778) (layer "F.Cu") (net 7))
 (segment (start 160.355739 107.018482) (end 160.295213 107.047629) (width 0.1778) (layer "F.Cu") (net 7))
 (segment (start 160.737988 107.400731) (end 160.752936 107.335237) (width 0.1778) (layer "F.Cu") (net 7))
 (segment (start 159.636309 106.858005) (end 159.678195 106.805482) (width 0.1778) (layer "F.Cu") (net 7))
 (segment (start 159.904407 106.486708) (end 159.904407 106.419529) (width 0.1778) (layer "F.Cu") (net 7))
 (segment (start 159.201407 106.423102) (end 159.140881 106.45225) (width 0.1778) (layer "F.Cu") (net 7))
 (segment (start 160.737988 107.202563) (end 160.70884 107.142038) (width 0.1778) (layer "F.Cu") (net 7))
 (segment (start 158.724175 105.306475) (end 158.658681 105.321424) (width 0.1778) (layer "F.Cu") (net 7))
 (segment (start 160.484838 108.025753) (end 160.455691 107.965227) (width 0.1778) (layer "F.Cu") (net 7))
 (segment (start 158.545632 105.392457) (end 158.4054 105.532688) (width 0.1778) (layer "F.Cu") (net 7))
 (segment (start 156.1592 98.605352) (end 158.779352 95.9852) (width 0.1778) (layer "F.Cu") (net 6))
 (segment (start 160.951801 95.9852) (end 161.274001 95.663) (width 0.1778) (layer "F.Cu") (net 6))
 (segment (start 158.779352 95.9852) (end 160.951801 95.9852) (width 0.1778) (layer "F.Cu") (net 6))
 (segment (start 164.465 108.901733) (end 163.460933 109.9058) (width 0.1778) (layer "F.Cu") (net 6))
 (segment (start 156.1592 104.213648) (end 156.1592 98.605352) (width 0.1778) (layer "F.Cu") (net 6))
 (segment (start 161.851352 109.9058) (end 156.1592 104.213648) (width 0.1778) (layer "F.Cu") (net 6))
 (segment (start 164.465 107.529) (end 164.465 108.901733) (width 0.1778) (layer "F.Cu") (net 6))
 (segment (start 163.460933 109.9058) (end 161.851352 109.9058) (width 0.1778) (layer "F.Cu") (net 6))
 (segment (start 163.362 106.426) (end 164.465 107.529) (width 0.1778) (layer "F.Cu") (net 6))
 (segment (start 161.274001 95.663) (end 161.274001 95.662999) (width 0.1778) (layer "F.Cu") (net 6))
 (segment (start 167.386 100.457) (end 166.243 101.6) (width 0.2032) (layer "F.Cu") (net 3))
 (segment (start 165.274 95.662999) (end 165.683702 95.662999) (width 0.2032) (layer "F.Cu") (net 3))
 (segment (start 167.386 97.365297) (end 167.386 100.457) (width 0.2032) (layer "F.Cu") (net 3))
 (segment (start 165.683702 95.662999) (end 167.386 97.365297) (width 0.2032) (layer "F.Cu") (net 3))
 (segment (start 166.274001 99.028999) (end 163.703 101.6) (width 0.2032) (layer "F.Cu") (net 2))
 (segment (start 166.274001 97.663) (end 166.274001 99.028999) (width 0.2032) (layer "F.Cu") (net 2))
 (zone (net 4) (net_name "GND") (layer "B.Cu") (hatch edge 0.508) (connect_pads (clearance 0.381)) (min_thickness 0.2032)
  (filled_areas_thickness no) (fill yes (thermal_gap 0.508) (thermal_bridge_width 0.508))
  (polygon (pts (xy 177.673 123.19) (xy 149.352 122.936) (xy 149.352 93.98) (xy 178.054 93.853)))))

